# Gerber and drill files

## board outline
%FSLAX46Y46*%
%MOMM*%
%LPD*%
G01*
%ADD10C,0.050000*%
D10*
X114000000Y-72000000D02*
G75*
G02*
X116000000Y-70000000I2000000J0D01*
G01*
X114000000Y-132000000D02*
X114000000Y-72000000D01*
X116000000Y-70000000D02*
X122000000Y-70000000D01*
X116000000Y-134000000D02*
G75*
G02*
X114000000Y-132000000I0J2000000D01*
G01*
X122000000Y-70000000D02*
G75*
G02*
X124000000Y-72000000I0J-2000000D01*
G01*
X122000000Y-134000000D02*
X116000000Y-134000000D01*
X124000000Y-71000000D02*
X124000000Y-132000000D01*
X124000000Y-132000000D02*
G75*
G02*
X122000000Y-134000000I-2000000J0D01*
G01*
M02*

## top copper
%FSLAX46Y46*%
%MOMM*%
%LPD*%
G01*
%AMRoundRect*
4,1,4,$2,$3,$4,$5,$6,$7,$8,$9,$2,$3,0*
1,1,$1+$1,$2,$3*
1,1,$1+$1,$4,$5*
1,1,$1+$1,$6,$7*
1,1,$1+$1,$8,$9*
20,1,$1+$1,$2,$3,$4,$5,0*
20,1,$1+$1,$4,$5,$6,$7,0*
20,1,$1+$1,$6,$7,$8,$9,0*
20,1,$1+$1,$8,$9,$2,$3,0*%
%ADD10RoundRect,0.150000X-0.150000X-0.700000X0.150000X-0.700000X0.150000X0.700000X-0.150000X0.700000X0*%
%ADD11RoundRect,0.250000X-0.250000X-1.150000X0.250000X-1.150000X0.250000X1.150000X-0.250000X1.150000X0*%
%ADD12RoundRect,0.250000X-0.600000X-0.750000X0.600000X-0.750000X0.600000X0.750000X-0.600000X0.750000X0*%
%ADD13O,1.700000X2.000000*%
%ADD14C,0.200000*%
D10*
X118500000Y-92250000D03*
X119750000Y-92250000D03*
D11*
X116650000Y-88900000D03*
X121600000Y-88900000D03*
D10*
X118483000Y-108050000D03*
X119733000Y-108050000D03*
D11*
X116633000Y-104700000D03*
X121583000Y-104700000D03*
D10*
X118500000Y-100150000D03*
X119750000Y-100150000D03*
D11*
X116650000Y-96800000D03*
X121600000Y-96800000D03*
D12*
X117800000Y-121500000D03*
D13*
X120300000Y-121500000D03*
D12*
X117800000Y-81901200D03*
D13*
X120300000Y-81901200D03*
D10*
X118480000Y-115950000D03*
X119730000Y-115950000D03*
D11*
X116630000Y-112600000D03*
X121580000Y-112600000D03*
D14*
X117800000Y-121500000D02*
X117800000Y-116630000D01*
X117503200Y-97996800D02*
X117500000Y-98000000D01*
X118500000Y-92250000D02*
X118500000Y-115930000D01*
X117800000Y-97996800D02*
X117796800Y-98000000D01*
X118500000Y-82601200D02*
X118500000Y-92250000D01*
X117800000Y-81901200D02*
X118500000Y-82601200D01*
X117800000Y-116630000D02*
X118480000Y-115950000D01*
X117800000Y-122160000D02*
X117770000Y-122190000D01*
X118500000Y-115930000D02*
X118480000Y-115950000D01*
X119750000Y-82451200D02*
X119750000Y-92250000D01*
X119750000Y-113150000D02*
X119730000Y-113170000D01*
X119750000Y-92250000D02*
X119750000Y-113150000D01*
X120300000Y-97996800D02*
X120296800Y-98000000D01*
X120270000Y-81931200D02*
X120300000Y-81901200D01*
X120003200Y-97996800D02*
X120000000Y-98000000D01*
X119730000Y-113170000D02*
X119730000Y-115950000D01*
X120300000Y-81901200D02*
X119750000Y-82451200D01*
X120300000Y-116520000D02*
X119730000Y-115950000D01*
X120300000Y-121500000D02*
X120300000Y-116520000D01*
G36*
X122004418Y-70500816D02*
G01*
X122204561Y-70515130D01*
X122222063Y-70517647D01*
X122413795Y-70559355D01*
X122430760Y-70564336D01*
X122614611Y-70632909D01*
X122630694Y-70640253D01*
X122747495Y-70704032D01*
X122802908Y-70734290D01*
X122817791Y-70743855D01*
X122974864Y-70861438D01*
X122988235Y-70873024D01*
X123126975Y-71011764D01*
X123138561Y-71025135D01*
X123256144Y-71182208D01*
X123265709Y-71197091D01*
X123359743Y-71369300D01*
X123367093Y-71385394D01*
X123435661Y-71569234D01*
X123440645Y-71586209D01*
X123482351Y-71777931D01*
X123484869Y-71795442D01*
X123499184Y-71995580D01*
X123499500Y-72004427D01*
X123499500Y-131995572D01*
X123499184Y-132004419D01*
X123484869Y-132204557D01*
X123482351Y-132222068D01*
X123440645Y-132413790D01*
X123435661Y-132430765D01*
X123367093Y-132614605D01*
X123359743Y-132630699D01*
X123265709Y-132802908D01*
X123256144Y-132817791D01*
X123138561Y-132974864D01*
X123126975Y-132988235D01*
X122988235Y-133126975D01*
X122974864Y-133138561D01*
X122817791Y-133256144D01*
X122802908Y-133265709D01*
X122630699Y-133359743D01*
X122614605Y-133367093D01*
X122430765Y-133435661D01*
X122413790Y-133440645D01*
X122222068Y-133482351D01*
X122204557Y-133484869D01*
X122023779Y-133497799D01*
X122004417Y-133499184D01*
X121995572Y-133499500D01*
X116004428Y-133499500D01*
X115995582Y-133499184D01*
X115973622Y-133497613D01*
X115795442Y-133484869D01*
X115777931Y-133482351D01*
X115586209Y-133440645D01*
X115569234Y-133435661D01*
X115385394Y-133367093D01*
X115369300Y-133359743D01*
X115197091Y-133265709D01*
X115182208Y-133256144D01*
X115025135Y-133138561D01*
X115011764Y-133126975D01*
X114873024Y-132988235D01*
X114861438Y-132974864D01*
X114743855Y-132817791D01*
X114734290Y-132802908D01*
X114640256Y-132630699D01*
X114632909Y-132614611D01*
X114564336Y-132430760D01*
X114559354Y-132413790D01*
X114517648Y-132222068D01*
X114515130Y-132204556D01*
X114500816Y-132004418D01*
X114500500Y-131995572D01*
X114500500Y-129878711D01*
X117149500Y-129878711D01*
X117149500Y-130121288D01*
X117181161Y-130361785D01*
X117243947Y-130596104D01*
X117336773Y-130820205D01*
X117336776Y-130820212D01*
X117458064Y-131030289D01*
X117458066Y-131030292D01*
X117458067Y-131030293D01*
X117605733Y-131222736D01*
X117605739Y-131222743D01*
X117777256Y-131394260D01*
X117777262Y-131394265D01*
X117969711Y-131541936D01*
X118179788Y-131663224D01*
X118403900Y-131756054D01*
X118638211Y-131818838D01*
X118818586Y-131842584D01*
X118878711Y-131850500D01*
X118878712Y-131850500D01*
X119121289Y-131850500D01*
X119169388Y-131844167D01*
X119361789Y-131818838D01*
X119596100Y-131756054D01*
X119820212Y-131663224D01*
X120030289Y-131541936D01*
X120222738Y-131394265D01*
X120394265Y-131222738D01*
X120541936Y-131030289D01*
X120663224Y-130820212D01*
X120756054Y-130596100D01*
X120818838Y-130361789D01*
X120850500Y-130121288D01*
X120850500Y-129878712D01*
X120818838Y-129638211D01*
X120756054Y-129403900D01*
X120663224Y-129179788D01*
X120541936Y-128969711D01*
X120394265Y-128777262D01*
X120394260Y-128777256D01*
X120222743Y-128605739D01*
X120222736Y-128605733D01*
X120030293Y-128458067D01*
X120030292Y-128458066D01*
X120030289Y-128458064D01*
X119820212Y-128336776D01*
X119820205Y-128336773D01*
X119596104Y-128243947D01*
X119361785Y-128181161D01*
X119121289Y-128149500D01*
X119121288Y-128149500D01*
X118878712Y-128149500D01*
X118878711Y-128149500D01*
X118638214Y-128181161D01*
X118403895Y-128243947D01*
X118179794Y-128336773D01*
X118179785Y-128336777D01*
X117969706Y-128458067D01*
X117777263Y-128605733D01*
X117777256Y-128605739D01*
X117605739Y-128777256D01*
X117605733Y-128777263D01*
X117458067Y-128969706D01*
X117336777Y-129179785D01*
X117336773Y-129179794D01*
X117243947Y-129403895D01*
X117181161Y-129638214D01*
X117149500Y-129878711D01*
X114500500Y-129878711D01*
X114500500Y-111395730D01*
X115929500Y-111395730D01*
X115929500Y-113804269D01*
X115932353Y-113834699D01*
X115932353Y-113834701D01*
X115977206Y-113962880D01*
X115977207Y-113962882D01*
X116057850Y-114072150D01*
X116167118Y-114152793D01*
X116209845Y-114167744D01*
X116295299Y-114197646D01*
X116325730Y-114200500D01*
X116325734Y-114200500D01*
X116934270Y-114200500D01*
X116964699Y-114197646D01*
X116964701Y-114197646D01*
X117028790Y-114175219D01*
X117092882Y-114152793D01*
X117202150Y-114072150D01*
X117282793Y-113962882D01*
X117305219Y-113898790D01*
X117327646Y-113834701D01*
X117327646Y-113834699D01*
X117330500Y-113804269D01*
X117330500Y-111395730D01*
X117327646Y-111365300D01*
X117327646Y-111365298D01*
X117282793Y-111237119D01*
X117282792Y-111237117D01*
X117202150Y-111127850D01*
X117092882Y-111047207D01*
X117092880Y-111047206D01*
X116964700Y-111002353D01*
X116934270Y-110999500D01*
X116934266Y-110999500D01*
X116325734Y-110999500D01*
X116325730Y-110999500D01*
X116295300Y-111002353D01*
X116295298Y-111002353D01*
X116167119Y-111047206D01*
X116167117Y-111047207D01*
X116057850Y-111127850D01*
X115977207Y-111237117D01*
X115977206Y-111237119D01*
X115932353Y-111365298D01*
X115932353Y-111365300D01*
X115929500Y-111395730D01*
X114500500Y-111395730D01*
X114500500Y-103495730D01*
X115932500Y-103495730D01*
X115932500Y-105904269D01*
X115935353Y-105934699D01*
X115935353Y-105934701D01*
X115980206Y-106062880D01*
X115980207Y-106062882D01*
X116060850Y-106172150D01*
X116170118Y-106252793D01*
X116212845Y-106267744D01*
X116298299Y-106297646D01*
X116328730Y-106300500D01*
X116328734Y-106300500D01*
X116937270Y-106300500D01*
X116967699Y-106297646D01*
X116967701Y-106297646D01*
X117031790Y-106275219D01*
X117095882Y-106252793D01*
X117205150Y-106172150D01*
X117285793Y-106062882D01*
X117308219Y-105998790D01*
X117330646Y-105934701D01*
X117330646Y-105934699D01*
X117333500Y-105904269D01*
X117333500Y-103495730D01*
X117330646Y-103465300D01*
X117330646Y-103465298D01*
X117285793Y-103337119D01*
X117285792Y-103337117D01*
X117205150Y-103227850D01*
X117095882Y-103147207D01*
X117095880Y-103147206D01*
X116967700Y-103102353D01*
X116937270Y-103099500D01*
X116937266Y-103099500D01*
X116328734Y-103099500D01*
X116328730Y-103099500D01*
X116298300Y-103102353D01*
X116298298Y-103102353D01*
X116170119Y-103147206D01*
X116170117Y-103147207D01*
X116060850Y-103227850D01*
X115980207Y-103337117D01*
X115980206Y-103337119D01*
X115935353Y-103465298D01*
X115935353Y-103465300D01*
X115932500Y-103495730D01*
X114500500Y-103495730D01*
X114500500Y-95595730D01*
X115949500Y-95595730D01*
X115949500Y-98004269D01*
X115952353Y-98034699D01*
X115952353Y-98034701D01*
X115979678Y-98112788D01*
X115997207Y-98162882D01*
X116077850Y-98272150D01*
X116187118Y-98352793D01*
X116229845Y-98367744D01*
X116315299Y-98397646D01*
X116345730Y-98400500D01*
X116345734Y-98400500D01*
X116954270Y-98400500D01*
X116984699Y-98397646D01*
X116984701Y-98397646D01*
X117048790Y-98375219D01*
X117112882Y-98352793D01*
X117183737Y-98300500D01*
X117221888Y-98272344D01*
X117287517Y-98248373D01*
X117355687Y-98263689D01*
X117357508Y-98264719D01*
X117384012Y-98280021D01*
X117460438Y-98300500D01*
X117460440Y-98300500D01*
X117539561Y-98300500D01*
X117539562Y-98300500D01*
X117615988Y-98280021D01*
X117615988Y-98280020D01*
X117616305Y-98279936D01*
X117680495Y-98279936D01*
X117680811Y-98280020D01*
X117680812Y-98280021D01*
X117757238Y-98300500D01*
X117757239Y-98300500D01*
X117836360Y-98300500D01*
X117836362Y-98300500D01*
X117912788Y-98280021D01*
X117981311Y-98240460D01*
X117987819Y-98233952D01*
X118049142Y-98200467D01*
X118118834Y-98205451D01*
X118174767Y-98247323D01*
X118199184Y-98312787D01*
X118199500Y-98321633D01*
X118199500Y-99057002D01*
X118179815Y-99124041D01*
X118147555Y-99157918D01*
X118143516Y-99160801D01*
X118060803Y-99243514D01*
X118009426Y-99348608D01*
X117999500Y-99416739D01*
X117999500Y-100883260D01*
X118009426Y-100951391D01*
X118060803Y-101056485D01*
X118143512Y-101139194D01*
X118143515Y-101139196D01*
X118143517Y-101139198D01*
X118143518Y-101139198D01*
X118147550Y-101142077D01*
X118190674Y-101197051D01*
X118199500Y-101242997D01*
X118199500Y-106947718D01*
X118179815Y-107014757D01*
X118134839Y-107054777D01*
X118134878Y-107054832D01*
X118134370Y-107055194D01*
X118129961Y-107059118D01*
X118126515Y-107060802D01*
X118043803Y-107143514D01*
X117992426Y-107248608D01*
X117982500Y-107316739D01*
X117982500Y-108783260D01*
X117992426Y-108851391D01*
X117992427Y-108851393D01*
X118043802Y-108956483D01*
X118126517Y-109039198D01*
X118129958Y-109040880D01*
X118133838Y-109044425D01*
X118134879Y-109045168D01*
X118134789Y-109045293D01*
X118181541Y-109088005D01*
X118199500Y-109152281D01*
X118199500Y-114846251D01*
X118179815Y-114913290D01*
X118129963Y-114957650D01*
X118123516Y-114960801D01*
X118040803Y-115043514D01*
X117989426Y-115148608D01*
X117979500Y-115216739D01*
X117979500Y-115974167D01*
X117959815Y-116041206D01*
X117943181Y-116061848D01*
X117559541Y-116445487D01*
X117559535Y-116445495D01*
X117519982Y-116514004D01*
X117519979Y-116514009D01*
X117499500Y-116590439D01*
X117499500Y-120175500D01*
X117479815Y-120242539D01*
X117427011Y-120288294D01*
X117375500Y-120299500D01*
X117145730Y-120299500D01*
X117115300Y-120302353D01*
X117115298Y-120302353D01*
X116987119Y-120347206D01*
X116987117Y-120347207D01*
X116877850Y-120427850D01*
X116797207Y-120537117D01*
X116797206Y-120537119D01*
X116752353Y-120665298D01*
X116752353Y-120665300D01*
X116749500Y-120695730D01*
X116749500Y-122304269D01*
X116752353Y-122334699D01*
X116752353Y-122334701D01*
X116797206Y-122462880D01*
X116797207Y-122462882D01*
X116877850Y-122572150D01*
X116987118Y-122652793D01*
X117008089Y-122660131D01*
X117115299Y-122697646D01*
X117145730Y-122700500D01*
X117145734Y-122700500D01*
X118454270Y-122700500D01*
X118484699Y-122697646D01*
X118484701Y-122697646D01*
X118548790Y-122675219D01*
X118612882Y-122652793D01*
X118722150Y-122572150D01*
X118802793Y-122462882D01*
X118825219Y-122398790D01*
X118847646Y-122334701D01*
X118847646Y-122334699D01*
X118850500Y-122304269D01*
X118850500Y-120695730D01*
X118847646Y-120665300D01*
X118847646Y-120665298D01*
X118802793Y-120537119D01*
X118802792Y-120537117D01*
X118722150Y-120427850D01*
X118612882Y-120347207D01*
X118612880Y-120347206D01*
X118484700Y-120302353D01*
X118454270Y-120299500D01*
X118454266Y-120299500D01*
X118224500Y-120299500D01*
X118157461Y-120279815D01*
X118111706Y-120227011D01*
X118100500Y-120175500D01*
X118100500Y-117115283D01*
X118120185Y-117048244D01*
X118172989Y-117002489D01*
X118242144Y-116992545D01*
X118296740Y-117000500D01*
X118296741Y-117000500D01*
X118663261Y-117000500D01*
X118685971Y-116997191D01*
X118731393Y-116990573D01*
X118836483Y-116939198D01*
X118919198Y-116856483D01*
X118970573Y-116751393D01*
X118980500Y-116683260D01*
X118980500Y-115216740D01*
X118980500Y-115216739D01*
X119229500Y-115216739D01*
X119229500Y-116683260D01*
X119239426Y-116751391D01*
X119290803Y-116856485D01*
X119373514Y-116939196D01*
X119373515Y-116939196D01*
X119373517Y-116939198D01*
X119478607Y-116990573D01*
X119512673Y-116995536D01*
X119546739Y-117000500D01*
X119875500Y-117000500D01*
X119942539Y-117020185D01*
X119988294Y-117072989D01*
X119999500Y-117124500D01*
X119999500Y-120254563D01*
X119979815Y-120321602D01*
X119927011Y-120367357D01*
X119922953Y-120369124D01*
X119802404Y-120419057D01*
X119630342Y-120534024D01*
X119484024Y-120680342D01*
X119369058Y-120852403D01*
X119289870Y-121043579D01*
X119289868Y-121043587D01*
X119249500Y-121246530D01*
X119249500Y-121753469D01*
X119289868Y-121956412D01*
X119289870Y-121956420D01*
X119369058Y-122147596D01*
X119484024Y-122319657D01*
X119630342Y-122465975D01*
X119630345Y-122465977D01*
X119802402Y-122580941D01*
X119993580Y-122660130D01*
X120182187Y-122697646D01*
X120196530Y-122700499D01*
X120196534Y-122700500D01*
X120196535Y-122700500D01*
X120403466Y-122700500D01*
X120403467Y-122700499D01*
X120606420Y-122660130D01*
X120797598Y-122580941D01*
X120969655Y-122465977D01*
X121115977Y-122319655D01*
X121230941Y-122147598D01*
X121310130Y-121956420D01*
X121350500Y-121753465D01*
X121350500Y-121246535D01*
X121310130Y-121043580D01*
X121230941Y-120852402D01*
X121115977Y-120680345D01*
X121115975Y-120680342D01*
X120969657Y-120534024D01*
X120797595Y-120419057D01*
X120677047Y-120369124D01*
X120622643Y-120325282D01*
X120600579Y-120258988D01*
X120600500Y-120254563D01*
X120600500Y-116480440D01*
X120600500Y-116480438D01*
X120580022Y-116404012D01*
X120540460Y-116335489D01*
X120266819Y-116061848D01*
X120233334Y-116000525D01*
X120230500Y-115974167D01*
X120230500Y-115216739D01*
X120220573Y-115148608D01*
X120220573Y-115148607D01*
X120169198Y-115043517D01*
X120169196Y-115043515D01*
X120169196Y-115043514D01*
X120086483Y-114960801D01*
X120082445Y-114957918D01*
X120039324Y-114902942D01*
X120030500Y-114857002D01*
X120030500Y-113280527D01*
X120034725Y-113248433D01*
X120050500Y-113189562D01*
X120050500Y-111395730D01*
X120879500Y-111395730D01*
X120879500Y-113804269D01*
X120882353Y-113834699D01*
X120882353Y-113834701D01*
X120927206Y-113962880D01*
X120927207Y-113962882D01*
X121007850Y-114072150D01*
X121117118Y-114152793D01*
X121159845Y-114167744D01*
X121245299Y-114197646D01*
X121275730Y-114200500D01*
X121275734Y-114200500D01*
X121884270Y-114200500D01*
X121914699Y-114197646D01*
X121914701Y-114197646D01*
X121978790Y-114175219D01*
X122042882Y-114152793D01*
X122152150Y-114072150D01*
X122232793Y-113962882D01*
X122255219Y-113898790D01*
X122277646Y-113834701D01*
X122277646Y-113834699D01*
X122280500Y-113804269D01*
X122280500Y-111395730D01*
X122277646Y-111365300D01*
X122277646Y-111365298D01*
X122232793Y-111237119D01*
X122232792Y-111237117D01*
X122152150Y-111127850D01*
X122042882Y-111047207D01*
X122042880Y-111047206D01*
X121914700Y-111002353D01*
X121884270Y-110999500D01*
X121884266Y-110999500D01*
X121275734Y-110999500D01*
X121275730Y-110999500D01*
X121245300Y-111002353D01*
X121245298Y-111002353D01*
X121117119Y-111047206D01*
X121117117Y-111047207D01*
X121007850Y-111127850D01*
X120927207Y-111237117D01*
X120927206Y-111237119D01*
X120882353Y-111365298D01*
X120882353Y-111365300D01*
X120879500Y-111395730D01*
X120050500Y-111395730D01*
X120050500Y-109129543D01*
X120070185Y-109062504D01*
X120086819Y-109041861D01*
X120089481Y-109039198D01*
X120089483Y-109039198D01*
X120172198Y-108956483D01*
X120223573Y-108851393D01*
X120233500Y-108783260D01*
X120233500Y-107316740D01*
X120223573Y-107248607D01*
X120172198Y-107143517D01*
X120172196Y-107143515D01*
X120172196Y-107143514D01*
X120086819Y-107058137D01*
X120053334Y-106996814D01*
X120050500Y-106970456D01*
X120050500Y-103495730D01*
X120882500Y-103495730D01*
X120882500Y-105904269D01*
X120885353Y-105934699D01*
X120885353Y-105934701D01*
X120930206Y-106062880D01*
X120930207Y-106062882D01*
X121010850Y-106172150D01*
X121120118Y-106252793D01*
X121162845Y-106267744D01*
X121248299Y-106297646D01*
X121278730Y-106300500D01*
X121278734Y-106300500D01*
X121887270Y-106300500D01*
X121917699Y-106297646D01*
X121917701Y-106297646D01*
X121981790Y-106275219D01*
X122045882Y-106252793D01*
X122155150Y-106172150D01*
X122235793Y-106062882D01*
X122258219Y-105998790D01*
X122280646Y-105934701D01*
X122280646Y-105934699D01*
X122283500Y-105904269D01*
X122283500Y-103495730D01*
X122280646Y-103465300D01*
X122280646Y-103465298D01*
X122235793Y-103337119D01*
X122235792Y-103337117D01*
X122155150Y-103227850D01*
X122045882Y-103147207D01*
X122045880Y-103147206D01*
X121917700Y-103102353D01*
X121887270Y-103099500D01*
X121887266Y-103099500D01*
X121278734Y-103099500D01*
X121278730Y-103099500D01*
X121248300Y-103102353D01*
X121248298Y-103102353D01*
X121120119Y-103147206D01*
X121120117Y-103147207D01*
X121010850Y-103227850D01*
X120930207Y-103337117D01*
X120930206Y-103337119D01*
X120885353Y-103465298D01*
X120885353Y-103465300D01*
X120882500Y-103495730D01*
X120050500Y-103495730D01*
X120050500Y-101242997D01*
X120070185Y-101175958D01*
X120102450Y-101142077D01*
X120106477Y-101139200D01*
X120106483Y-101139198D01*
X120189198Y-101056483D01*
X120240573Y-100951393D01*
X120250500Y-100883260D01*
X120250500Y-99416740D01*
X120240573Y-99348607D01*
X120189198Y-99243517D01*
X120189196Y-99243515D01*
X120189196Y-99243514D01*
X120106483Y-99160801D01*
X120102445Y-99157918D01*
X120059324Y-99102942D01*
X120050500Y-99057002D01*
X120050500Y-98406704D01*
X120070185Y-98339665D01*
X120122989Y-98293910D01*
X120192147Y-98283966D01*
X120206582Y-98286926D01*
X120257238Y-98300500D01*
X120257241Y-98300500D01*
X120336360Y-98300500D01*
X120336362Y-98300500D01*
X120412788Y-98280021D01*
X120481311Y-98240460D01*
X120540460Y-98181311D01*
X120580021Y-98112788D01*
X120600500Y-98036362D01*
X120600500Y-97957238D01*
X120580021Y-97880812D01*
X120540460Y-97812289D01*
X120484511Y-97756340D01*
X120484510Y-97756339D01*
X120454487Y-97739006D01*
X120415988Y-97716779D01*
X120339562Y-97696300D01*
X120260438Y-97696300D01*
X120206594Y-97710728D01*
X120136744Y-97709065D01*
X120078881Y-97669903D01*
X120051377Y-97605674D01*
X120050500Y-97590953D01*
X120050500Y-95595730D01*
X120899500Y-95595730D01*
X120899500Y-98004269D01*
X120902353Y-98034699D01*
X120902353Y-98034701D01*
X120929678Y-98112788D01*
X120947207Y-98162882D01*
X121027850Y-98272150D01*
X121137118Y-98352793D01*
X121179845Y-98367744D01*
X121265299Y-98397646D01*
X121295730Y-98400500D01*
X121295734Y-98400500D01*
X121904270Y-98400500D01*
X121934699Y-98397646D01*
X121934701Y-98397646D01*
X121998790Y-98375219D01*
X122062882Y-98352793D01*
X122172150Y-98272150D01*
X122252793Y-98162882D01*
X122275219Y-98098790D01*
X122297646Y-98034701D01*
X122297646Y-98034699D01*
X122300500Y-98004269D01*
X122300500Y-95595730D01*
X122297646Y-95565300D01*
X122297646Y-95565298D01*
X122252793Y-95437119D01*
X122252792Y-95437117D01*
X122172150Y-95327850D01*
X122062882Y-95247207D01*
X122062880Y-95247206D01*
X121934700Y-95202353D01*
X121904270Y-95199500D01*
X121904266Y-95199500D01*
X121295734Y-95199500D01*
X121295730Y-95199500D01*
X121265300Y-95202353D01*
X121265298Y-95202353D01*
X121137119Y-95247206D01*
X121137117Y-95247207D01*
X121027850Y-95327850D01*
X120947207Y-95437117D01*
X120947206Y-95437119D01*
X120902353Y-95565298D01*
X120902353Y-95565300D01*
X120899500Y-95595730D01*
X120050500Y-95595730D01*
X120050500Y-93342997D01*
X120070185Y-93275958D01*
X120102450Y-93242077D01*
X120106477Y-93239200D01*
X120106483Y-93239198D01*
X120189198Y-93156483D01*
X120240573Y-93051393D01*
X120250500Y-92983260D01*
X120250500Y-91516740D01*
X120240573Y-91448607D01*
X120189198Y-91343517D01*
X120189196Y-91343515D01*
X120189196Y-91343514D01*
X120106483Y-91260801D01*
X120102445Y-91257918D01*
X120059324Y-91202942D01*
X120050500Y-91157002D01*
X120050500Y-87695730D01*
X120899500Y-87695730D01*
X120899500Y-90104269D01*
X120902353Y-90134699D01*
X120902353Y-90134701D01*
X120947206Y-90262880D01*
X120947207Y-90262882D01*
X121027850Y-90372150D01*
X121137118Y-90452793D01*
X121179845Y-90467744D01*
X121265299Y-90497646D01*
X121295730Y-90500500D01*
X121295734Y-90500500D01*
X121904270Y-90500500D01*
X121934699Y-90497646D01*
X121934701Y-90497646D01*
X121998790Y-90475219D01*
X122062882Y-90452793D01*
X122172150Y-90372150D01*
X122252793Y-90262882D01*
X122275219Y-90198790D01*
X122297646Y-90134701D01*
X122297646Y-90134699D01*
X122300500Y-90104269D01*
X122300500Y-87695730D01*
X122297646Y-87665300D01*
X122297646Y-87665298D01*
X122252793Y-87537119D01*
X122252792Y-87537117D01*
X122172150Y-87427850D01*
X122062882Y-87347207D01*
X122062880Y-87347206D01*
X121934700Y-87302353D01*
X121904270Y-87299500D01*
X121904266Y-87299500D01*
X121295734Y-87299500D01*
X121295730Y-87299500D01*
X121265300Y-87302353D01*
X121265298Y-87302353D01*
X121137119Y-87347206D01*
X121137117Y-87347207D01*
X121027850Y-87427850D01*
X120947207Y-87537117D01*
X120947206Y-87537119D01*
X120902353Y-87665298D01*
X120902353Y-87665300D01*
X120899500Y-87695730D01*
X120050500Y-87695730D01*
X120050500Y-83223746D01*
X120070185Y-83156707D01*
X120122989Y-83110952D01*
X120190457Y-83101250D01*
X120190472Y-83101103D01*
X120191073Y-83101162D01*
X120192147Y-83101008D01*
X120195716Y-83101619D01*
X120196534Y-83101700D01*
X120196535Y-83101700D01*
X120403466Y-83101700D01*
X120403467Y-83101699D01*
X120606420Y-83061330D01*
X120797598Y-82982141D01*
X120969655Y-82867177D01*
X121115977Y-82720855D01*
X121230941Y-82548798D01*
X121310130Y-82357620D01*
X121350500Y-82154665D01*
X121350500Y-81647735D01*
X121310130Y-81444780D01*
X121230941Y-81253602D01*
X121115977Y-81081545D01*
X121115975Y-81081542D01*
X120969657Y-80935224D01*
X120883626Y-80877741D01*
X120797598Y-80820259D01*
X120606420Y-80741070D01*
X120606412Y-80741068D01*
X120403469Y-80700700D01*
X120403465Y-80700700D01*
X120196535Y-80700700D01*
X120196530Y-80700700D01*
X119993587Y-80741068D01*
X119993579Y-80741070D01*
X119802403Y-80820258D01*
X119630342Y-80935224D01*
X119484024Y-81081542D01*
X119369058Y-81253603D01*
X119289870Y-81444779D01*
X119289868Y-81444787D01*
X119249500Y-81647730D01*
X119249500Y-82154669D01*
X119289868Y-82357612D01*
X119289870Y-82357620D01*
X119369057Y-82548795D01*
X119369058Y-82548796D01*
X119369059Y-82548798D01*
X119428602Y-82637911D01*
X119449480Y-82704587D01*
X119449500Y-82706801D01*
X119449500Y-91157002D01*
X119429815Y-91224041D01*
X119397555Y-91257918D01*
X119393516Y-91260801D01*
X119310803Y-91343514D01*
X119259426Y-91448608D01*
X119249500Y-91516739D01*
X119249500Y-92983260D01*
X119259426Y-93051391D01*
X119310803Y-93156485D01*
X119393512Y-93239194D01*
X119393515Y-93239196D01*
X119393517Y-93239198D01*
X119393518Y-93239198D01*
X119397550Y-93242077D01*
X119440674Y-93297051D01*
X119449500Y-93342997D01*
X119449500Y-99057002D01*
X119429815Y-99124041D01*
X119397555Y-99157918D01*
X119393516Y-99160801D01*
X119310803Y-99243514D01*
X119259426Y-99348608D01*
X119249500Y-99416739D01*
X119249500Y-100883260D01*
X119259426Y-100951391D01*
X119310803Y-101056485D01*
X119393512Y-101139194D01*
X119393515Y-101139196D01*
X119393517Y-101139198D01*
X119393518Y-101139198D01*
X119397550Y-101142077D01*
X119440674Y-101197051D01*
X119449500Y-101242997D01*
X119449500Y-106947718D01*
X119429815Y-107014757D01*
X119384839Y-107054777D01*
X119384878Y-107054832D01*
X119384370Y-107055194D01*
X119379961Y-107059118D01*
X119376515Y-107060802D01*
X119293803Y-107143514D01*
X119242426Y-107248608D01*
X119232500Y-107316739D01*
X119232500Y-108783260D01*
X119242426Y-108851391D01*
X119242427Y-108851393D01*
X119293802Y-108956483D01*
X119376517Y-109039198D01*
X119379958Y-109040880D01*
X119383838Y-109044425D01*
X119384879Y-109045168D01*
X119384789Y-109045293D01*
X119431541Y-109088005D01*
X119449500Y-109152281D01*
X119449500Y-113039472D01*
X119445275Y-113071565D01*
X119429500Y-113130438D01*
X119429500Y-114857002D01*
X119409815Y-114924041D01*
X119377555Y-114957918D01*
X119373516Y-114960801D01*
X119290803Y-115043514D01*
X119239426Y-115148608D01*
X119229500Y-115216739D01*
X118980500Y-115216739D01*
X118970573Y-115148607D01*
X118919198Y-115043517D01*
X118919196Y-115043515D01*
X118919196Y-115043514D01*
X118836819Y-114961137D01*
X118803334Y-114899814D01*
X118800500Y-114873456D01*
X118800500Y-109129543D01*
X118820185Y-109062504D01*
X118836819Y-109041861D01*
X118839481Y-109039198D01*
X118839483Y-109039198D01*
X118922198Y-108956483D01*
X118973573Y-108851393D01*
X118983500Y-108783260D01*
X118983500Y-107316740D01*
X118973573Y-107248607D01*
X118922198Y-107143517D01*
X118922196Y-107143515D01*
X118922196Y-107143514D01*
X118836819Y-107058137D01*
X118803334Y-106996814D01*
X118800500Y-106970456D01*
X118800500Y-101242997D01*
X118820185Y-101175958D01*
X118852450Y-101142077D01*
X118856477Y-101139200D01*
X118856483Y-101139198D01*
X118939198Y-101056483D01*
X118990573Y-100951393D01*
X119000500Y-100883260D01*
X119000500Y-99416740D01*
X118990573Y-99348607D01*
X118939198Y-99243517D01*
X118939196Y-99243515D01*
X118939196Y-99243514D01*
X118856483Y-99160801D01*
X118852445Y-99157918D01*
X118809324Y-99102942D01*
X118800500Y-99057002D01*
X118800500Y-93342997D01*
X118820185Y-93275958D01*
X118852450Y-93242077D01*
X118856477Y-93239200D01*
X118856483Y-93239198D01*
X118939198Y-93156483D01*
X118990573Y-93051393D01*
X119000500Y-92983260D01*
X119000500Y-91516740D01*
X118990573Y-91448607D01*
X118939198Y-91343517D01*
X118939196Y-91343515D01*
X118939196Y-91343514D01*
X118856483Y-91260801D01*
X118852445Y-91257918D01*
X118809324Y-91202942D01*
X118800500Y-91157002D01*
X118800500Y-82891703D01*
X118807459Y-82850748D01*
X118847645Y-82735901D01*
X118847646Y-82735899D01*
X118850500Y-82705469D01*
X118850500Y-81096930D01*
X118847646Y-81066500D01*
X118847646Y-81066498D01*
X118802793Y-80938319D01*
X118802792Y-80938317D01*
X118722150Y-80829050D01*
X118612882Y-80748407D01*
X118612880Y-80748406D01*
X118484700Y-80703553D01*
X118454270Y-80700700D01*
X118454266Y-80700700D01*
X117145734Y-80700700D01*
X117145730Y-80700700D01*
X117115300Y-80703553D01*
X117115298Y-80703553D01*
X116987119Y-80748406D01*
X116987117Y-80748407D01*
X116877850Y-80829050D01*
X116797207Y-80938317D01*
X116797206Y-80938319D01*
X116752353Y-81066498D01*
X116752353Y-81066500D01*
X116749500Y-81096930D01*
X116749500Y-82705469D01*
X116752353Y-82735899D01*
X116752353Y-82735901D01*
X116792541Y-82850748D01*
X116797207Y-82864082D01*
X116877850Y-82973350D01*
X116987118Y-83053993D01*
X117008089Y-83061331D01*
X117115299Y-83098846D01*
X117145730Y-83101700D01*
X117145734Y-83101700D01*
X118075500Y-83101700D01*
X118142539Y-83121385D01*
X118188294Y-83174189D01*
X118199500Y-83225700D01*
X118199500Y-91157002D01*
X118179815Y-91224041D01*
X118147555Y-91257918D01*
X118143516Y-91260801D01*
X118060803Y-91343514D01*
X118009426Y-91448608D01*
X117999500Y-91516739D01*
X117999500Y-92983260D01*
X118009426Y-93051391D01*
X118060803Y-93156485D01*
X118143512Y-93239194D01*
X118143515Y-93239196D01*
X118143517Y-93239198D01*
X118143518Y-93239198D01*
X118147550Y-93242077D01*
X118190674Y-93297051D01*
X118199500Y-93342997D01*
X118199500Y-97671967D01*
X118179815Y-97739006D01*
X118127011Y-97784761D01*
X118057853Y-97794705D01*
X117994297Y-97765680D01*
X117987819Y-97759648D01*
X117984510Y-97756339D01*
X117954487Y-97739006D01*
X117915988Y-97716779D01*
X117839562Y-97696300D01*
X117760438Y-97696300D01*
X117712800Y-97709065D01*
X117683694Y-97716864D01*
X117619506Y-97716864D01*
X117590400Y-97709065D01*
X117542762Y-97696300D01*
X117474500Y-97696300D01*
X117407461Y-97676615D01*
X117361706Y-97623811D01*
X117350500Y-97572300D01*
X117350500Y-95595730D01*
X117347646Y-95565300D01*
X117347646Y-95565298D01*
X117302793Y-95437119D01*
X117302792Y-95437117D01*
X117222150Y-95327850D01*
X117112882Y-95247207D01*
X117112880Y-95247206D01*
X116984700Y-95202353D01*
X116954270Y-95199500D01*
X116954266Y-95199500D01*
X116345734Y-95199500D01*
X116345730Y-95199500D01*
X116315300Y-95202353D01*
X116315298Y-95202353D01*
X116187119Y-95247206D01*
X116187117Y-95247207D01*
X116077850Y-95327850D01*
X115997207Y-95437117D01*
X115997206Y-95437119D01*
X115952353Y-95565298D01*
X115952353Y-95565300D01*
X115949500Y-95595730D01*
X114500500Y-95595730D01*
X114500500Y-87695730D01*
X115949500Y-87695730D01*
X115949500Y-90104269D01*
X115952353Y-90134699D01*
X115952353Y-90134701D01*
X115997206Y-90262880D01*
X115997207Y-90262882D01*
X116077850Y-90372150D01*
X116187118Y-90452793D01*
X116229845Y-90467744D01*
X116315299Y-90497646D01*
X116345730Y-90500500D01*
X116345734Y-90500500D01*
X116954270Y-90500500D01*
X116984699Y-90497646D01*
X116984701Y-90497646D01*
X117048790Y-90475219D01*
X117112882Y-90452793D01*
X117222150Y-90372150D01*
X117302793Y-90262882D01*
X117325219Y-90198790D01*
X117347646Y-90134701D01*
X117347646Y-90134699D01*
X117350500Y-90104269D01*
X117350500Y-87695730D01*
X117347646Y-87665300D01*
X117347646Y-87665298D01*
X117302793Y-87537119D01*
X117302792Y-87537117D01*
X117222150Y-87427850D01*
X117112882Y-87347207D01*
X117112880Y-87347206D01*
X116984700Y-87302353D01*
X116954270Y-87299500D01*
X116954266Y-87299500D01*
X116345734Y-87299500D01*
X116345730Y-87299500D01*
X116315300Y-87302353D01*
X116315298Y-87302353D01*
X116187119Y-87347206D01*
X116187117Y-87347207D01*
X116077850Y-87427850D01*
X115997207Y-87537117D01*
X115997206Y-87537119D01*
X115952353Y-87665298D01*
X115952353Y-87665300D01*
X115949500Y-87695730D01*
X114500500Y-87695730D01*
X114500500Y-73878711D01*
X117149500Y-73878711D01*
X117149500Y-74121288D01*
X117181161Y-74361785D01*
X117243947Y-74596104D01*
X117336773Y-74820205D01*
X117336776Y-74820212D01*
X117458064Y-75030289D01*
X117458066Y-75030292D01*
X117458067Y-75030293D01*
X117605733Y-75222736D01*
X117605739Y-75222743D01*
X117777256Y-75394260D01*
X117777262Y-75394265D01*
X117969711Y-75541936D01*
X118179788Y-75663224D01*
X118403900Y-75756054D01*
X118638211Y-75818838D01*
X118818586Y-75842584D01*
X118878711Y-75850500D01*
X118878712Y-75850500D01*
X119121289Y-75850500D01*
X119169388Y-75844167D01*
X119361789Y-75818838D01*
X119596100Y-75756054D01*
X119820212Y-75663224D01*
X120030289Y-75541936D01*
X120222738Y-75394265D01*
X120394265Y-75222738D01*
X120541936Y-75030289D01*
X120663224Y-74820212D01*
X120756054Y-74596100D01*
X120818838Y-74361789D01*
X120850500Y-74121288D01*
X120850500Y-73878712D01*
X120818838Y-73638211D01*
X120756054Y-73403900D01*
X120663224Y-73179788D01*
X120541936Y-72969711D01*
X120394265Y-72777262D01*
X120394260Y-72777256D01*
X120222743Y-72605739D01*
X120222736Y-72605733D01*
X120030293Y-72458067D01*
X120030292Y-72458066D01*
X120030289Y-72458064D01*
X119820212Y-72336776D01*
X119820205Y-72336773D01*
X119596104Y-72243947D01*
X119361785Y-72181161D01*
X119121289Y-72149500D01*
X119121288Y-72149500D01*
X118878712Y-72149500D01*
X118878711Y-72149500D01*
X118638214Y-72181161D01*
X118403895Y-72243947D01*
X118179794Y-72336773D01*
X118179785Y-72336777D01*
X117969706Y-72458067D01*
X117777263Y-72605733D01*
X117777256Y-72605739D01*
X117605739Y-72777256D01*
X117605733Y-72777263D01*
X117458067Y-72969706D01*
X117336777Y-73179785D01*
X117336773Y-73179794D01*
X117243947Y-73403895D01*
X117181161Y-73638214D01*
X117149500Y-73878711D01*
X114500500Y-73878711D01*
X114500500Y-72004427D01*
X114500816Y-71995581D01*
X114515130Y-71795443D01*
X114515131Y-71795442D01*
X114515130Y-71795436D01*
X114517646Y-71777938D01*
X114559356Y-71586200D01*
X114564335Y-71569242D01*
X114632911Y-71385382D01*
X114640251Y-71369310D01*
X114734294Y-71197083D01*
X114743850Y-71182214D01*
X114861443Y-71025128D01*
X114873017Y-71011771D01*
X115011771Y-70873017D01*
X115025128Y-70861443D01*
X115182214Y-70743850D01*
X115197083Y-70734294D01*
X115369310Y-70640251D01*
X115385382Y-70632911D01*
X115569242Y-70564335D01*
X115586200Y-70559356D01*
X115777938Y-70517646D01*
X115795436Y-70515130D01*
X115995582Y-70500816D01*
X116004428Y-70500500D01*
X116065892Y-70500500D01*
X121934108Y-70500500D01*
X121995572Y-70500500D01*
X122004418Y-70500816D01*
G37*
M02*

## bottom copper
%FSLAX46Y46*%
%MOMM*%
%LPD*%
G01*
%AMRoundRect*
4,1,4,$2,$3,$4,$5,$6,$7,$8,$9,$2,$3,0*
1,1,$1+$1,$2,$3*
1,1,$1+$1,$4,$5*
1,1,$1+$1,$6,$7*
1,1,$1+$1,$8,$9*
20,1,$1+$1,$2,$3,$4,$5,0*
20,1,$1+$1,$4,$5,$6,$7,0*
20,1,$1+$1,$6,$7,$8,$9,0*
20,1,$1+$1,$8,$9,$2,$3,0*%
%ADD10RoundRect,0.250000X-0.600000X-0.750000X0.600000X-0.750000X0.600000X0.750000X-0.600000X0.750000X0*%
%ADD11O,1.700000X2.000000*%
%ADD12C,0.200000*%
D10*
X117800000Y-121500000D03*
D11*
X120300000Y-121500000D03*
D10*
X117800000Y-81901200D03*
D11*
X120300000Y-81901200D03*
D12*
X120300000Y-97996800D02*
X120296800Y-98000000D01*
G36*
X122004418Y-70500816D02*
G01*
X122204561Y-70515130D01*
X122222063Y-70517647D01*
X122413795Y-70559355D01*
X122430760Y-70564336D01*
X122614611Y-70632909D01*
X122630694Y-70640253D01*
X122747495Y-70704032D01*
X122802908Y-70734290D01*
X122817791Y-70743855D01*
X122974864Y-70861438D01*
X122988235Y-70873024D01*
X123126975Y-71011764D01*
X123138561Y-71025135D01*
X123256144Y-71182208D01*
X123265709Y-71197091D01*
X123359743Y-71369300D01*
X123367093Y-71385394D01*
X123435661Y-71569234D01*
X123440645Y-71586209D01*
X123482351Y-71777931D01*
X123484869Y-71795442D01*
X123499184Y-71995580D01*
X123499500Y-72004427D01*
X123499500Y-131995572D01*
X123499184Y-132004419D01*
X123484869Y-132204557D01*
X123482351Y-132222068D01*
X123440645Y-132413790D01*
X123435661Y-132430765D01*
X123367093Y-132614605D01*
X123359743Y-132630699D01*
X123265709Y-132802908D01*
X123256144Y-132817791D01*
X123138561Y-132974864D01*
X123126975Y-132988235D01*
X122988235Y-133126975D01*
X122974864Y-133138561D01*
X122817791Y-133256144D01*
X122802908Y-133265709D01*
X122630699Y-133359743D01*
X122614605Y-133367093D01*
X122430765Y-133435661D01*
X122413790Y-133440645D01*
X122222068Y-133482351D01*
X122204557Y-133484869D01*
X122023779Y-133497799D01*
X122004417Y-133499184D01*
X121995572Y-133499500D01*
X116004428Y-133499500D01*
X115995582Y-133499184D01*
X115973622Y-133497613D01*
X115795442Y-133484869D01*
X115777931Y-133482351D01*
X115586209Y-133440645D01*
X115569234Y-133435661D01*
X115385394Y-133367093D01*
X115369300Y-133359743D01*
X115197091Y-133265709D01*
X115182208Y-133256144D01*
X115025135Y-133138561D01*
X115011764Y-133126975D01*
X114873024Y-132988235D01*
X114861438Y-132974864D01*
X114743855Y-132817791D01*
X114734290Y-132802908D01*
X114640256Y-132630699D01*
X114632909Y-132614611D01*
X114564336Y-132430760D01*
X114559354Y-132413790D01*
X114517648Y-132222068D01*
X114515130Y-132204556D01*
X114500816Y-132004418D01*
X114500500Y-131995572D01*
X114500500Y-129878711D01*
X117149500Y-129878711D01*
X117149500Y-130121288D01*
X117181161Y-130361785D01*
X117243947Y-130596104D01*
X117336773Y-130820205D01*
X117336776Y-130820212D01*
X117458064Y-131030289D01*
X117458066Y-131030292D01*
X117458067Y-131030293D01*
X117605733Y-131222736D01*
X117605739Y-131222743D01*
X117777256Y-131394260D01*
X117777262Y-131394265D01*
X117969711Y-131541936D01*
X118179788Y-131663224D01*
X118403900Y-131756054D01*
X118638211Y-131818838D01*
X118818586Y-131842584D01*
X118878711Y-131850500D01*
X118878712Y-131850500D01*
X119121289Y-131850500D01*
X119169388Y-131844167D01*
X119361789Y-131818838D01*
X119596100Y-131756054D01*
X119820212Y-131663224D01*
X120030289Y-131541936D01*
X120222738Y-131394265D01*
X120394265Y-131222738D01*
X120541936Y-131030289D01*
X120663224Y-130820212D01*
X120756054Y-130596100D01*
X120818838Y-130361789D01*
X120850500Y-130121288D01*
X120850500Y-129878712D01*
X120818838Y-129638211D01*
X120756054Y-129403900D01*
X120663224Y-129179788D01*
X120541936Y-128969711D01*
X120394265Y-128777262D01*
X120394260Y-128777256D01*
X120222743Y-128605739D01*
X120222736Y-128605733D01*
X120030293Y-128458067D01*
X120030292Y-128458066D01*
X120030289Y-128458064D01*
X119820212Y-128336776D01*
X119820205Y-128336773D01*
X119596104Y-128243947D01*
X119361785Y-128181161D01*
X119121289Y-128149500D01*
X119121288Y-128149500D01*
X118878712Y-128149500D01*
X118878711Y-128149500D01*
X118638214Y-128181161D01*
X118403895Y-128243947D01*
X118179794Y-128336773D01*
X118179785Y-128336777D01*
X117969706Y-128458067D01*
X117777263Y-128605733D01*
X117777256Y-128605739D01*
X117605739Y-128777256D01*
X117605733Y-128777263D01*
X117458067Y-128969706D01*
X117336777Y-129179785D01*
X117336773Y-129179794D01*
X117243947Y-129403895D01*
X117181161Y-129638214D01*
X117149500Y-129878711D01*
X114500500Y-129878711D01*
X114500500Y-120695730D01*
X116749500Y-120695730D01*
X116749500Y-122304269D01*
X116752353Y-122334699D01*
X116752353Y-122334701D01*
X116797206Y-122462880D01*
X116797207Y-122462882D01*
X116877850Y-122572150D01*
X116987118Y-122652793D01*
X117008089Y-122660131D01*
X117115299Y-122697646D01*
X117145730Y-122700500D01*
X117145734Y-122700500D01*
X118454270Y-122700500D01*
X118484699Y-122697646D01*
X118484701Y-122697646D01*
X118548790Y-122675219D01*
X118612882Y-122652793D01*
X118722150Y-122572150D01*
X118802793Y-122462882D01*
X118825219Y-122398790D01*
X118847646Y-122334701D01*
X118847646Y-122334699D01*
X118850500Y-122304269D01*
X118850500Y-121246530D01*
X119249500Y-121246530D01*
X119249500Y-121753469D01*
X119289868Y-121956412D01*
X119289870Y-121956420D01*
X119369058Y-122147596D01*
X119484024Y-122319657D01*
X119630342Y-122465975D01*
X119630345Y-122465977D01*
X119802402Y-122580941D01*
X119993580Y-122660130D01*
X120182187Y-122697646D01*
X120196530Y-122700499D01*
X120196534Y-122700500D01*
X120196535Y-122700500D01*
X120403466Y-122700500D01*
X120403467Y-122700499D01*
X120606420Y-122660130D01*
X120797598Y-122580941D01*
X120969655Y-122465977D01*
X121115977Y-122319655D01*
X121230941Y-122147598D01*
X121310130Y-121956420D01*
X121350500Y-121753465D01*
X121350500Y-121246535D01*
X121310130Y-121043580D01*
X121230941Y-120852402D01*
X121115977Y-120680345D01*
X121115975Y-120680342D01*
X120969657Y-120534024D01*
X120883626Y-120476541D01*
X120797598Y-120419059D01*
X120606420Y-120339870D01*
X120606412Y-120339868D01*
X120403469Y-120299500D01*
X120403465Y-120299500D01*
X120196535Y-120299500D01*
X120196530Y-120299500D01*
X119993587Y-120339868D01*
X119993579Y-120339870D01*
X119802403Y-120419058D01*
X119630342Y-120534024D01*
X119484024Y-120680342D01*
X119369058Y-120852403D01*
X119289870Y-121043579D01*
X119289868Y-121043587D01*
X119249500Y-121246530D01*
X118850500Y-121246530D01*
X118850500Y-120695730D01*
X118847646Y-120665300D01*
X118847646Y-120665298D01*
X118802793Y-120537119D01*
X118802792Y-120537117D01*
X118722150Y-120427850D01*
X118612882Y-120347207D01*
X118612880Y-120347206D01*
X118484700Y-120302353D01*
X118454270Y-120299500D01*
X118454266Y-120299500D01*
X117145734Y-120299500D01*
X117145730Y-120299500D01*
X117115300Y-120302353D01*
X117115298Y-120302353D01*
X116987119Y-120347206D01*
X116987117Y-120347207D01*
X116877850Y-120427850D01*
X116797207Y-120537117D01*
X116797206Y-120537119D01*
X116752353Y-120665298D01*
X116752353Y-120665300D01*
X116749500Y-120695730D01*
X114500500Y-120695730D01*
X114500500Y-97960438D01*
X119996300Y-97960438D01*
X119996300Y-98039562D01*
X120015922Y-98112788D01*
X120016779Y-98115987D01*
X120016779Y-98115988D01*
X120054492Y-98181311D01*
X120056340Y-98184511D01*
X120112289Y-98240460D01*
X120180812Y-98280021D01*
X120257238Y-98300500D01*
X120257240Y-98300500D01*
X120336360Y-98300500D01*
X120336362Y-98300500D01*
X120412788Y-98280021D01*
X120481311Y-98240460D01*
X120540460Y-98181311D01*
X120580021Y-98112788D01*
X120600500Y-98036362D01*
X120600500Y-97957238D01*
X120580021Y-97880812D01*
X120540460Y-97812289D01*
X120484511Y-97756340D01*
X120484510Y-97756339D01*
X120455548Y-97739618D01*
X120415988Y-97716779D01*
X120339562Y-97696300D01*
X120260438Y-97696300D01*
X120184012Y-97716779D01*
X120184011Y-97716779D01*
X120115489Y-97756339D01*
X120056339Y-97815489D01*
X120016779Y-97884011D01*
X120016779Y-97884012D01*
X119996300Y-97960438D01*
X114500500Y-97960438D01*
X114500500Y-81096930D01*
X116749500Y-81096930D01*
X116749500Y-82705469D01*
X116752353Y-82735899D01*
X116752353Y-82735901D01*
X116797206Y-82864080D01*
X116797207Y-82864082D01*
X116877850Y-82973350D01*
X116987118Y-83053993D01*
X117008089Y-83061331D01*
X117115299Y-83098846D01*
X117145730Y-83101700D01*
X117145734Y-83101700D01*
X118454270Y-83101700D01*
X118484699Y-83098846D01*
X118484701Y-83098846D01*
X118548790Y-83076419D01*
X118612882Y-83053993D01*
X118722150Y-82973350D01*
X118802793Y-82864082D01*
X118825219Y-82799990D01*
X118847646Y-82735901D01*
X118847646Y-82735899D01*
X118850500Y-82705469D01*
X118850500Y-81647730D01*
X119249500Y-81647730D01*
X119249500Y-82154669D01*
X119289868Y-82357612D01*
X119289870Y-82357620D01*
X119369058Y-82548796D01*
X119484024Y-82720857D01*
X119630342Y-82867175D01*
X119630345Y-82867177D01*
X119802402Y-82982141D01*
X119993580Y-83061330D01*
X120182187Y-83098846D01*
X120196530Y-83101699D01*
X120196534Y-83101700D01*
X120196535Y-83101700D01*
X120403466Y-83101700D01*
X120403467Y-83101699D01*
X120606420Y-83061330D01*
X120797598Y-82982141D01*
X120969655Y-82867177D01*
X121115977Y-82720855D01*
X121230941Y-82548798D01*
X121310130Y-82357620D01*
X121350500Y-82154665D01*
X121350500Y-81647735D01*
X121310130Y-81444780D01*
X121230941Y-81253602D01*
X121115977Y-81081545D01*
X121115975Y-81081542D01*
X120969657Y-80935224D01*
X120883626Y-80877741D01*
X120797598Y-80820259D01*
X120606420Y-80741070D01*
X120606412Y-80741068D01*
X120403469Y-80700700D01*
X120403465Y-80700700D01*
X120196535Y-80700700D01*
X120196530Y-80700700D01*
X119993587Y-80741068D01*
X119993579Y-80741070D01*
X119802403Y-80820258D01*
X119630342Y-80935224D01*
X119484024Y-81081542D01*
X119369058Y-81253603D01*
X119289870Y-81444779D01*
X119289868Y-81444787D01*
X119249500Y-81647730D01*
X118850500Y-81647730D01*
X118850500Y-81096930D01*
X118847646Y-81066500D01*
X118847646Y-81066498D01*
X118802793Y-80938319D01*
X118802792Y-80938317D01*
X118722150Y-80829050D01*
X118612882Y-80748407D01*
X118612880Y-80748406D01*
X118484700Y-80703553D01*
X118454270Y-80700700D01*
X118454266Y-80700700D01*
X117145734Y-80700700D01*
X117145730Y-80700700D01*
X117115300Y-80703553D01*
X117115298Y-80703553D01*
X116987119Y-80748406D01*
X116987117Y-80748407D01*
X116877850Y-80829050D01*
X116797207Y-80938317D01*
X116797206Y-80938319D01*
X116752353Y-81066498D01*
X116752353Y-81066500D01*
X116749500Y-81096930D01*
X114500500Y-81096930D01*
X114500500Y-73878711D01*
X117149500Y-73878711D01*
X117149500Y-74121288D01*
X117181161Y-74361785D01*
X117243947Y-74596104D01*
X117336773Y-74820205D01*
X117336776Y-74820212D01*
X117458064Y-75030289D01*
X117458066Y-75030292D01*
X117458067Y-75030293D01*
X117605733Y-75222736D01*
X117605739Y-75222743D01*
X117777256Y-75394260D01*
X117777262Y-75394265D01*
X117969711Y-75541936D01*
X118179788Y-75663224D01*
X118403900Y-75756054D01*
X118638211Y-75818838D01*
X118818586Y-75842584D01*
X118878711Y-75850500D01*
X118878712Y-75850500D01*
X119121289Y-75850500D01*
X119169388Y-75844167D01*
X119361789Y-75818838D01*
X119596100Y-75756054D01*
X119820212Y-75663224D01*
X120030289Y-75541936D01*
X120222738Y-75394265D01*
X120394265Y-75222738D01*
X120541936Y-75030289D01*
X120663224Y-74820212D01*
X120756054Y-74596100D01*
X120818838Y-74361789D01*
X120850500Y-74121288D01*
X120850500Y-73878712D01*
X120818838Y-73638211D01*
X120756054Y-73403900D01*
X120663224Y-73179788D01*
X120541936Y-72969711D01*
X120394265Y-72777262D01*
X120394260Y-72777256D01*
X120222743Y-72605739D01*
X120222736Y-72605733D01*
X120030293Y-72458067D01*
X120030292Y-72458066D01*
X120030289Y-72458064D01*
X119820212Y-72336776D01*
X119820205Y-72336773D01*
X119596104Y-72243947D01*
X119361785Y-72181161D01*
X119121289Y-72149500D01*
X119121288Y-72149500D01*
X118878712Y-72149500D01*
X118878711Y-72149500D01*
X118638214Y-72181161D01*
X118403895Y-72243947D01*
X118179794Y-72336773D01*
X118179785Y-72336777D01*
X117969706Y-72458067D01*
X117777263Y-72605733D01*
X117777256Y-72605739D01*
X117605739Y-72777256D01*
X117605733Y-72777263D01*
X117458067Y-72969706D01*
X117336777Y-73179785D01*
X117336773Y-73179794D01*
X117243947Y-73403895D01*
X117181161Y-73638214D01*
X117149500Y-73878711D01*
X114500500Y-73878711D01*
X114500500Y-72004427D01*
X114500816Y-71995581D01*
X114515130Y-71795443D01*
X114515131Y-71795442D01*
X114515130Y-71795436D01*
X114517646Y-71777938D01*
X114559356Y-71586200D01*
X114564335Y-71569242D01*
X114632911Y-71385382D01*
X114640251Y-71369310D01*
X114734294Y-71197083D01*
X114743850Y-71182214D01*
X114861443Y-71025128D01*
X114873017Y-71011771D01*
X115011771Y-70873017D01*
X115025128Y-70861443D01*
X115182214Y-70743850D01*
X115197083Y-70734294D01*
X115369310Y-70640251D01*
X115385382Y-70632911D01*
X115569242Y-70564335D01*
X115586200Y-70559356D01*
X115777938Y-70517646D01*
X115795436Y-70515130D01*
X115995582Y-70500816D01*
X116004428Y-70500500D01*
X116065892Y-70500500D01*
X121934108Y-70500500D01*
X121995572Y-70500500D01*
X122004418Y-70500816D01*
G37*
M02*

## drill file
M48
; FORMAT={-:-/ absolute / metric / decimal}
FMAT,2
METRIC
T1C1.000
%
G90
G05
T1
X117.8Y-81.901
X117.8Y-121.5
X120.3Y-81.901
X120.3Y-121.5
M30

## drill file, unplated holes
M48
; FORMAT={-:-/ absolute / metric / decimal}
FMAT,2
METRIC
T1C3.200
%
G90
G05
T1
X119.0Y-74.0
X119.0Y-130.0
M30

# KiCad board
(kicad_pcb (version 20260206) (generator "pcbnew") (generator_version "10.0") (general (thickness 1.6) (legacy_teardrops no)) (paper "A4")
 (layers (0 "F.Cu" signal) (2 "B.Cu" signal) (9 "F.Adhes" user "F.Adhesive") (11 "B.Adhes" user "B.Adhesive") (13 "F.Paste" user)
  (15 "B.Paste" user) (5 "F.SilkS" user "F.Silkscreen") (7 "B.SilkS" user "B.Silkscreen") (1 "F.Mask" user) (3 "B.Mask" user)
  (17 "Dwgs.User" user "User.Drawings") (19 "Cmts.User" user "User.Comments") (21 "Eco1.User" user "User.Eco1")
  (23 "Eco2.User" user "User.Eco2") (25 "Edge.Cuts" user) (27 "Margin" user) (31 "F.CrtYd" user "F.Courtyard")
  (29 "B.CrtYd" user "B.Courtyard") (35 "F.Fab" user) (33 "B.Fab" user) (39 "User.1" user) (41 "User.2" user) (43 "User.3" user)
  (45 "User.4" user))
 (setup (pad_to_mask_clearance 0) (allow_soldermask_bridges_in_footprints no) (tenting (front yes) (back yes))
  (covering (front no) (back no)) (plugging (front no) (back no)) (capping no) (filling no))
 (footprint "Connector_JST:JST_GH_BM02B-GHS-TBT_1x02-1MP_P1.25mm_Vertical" (layer "F.Cu") (at 119.125 90.3)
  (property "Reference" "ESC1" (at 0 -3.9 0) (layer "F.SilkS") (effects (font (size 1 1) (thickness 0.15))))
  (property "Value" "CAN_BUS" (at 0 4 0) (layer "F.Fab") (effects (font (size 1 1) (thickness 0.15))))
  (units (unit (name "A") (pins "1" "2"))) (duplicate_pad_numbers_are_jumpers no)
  (pad "1" smd roundrect (at -0.625 1.95) (size 0.6 1.7) (layers "F.Cu" "F.Mask" "F.Paste") (roundrect_rratio 0.25) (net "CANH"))
  (pad "2" smd roundrect (at 0.625 1.95) (size 0.6 1.7) (layers "F.Cu" "F.Mask" "F.Paste") (roundrect_rratio 0.25) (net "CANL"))
  (pad "MP" smd roundrect (at -2.475 -1.4) (size 1 2.8) (layers "F.Cu" "F.Mask" "F.Paste") (roundrect_rratio 0.25))
  (pad "MP" smd roundrect (at 2.475 -1.4) (size 1 2.8) (layers "F.Cu" "F.Mask" "F.Paste") (roundrect_rratio 0.25)))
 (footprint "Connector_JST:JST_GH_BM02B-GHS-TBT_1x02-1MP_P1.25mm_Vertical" (layer "F.Cu") (at 119.108 106.1)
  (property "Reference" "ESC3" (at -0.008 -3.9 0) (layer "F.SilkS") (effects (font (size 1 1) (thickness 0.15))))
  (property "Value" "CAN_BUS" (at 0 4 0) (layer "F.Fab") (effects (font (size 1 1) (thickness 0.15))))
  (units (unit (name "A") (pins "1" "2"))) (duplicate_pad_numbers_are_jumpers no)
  (pad "1" smd roundrect (at -0.625 1.95) (size 0.6 1.7) (layers "F.Cu" "F.Mask" "F.Paste") (roundrect_rratio 0.25) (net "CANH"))
  (pad "2" smd roundrect (at 0.625 1.95) (size 0.6 1.7) (layers "F.Cu" "F.Mask" "F.Paste") (roundrect_rratio 0.25) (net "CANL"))
  (pad "MP" smd roundrect (at -2.475 -1.4) (size 1 2.8) (layers "F.Cu" "F.Mask" "F.Paste") (roundrect_rratio 0.25))
  (pad "MP" smd roundrect (at 2.475 -1.4) (size 1 2.8) (layers "F.Cu" "F.Mask" "F.Paste") (roundrect_rratio 0.25)))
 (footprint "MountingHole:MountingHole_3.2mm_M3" (layer "F.Cu") (at 119 130)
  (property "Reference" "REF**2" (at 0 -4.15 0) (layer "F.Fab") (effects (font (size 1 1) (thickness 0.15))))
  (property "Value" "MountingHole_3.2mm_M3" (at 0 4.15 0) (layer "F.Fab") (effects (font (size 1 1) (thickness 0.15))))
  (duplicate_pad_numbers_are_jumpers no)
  (pad "" np_thru_hole circle (at 0 0) (size 3.2 3.2) (drill 3.2) (layers "*.Cu" "*.Mask")))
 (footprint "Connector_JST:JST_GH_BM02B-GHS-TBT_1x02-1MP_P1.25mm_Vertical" (layer "F.Cu") (at 119.125 98.2)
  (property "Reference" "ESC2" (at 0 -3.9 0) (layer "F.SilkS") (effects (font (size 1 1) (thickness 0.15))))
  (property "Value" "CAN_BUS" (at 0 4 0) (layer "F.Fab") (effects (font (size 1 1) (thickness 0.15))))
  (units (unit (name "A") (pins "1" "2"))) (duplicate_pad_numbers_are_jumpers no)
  (pad "1" smd roundrect (at -0.625 1.95) (size 0.6 1.7) (layers "F.Cu" "F.Mask" "F.Paste") (roundrect_rratio 0.25) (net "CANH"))
  (pad "2" smd roundrect (at 0.625 1.95) (size 0.6 1.7) (layers "F.Cu" "F.Mask" "F.Paste") (roundrect_rratio 0.25) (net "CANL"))
  (pad "MP" smd roundrect (at -2.475 -1.4) (size 1 2.8) (layers "F.Cu" "F.Mask" "F.Paste") (roundrect_rratio 0.25))
  (pad "MP" smd roundrect (at 2.475 -1.4) (size 1 2.8) (layers "F.Cu" "F.Mask" "F.Paste") (roundrect_rratio 0.25)))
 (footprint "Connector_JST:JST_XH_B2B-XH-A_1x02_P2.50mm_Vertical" (layer "F.Cu") (at 117.8 121.5)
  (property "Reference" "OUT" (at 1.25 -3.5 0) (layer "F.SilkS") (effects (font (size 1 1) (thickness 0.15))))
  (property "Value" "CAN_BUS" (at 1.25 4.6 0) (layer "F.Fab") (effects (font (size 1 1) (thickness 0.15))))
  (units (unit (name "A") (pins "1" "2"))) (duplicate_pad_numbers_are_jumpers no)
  (pad "1" thru_hole roundrect (at 0 0) (size 1.7 2) (drill 1) (layers "*.Cu" "*.Mask") (remove_unused_layers no)
   (roundrect_rratio 0.147059) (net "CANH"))
  (pad "2" thru_hole oval (at 2.5 0) (size 1.7 2) (drill 1) (layers "*.Cu" "*.Mask") (remove_unused_layers no) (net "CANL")))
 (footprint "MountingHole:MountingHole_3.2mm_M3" (layer "F.Cu") (at 119 74)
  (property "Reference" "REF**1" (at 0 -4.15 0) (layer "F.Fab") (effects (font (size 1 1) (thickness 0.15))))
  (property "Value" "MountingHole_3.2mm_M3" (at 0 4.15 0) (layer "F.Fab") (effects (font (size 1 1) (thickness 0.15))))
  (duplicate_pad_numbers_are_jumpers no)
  (pad "" np_thru_hole circle (at 0 0) (size 3.2 3.2) (drill 3.2) (layers "*.Cu" "*.Mask")))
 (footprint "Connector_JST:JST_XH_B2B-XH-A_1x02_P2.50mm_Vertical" (layer "F.Cu") (at 117.8 81.9012)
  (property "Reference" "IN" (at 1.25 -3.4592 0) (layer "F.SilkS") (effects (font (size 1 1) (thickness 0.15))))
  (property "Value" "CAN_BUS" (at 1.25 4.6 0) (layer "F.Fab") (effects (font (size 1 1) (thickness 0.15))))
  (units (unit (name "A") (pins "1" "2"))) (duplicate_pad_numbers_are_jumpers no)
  (pad "1" thru_hole roundrect (at 0 0) (size 1.7 2) (drill 1) (layers "*.Cu" "*.Mask") (remove_unused_layers no)
   (roundrect_rratio 0.147059) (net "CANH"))
  (pad "2" thru_hole oval (at 2.5 0) (size 1.7 2) (drill 1) (layers "*.Cu" "*.Mask") (remove_unused_layers no) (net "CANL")))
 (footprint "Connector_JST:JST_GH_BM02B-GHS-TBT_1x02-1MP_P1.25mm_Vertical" (layer "F.Cu") (at 119.105 114)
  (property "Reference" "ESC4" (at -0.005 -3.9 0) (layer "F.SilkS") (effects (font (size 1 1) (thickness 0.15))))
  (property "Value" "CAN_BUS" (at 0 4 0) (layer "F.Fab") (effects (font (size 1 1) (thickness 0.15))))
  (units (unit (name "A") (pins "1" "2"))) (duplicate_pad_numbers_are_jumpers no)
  (pad "1" smd roundrect (at -0.625 1.95) (size 0.6 1.7) (layers "F.Cu" "F.Mask" "F.Paste") (roundrect_rratio 0.25) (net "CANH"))
  (pad "2" smd roundrect (at 0.625 1.95) (size 0.6 1.7) (layers "F.Cu" "F.Mask" "F.Paste") (roundrect_rratio 0.25) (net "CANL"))
  (pad "MP" smd roundrect (at -2.475 -1.4) (size 1 2.8) (layers "F.Cu" "F.Mask" "F.Paste") (roundrect_rratio 0.25))
  (pad "MP" smd roundrect (at 2.475 -1.4) (size 1 2.8) (layers "F.Cu" "F.Mask" "F.Paste") (roundrect_rratio 0.25)))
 (gr_arc (start 114 72) (mid 114.585786 70.585786) (end 116 70) (stroke (width 0.05) (type default)) (layer "Edge.Cuts"))
 (gr_line (start 114 132) (end 114 72) (stroke (width 0.05) (type default)) (layer "Edge.Cuts"))
 (gr_line (start 116 70) (end 122 70) (stroke (width 0.05) (type default)) (layer "Edge.Cuts"))
 (gr_arc (start 116 134) (mid 114.585786 133.414214) (end 114 132) (stroke (width 0.05) (type default)) (layer "Edge.Cuts"))
 (gr_arc (start 122 70) (mid 123.414214 70.585786) (end 124 72) (stroke (width 0.05) (type default)) (layer "Edge.Cuts"))
 (gr_line (start 122 134) (end 116 134) (stroke (width 0.05) (type default)) (layer "Edge.Cuts"))
 (gr_line (start 124 71) (end 124 132) (stroke (width 0.05) (type default)) (layer "Edge.Cuts"))
 (gr_arc (start 124 132) (mid 123.414214 133.414214) (end 122 134) (stroke (width 0.05) (type default)) (layer "Edge.Cuts"))
 (segment (start 117.8 121.5) (end 117.8 116.63) (width 0.2) (layer "F.Cu") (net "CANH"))
 (segment (start 117.5032 97.9968) (end 117.5 98) (width 0.2) (layer "F.Cu") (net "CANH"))
 (segment (start 118.5 92.25) (end 118.5 115.93) (width 0.2) (layer "F.Cu") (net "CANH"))
 (segment (start 117.8 97.9968) (end 117.7968 98) (width 0.2) (layer "F.Cu") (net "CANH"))
 (segment (start 118.5 82.6012) (end 118.5 92.25) (width 0.2) (layer "F.Cu") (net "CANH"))
 (segment (start 117.8 81.9012) (end 118.5 82.6012) (width 0.2) (layer "F.Cu") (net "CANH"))
 (segment (start 117.8 116.63) (end 118.48 115.95) (width 0.2) (layer "F.Cu") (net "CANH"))
 (segment (start 117.8 122.16) (end 117.77 122.19) (width 0.2) (layer "F.Cu") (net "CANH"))
 (segment (start 118.5 115.93) (end 118.48 115.95) (width 0.2) (layer "F.Cu") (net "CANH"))
 (segment (start 119.75 82.4512) (end 119.75 92.25) (width 0.2) (layer "F.Cu") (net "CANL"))
 (segment (start 119.75 113.15) (end 119.73 113.17) (width 0.2) (layer "F.Cu") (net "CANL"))
 (segment (start 119.75 92.25) (end 119.75 113.15) (width 0.2) (layer "F.Cu") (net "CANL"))
 (segment (start 120.3 97.9968) (end 120.2968 98) (width 0.2) (layer "F.Cu") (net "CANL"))
 (segment (start 120.27 81.9312) (end 120.3 81.9012) (width 0.2) (layer "F.Cu") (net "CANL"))
 (segment (start 120.0032 97.9968) (end 120 98) (width 0.2) (layer "F.Cu") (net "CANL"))
 (segment (start 119.73 113.17) (end 119.73 115.95) (width 0.2) (layer "F.Cu") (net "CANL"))
 (segment (start 120.3 81.9012) (end 119.75 82.4512) (width 0.2) (layer "F.Cu") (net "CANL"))
 (segment (start 120.3 116.52) (end 119.73 115.95) (width 0.2) (layer "F.Cu") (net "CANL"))
 (segment (start 120.3 121.5) (end 120.3 116.52) (width 0.2) (layer "F.Cu") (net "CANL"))
 (segment (start 120.3 97.9968) (end 120.2968 98) (width 0.2) (layer "B.Cu") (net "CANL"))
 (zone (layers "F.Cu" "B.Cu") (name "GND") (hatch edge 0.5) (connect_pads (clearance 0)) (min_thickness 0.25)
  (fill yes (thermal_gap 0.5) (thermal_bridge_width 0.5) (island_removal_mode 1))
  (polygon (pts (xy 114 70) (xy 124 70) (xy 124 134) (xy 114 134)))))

